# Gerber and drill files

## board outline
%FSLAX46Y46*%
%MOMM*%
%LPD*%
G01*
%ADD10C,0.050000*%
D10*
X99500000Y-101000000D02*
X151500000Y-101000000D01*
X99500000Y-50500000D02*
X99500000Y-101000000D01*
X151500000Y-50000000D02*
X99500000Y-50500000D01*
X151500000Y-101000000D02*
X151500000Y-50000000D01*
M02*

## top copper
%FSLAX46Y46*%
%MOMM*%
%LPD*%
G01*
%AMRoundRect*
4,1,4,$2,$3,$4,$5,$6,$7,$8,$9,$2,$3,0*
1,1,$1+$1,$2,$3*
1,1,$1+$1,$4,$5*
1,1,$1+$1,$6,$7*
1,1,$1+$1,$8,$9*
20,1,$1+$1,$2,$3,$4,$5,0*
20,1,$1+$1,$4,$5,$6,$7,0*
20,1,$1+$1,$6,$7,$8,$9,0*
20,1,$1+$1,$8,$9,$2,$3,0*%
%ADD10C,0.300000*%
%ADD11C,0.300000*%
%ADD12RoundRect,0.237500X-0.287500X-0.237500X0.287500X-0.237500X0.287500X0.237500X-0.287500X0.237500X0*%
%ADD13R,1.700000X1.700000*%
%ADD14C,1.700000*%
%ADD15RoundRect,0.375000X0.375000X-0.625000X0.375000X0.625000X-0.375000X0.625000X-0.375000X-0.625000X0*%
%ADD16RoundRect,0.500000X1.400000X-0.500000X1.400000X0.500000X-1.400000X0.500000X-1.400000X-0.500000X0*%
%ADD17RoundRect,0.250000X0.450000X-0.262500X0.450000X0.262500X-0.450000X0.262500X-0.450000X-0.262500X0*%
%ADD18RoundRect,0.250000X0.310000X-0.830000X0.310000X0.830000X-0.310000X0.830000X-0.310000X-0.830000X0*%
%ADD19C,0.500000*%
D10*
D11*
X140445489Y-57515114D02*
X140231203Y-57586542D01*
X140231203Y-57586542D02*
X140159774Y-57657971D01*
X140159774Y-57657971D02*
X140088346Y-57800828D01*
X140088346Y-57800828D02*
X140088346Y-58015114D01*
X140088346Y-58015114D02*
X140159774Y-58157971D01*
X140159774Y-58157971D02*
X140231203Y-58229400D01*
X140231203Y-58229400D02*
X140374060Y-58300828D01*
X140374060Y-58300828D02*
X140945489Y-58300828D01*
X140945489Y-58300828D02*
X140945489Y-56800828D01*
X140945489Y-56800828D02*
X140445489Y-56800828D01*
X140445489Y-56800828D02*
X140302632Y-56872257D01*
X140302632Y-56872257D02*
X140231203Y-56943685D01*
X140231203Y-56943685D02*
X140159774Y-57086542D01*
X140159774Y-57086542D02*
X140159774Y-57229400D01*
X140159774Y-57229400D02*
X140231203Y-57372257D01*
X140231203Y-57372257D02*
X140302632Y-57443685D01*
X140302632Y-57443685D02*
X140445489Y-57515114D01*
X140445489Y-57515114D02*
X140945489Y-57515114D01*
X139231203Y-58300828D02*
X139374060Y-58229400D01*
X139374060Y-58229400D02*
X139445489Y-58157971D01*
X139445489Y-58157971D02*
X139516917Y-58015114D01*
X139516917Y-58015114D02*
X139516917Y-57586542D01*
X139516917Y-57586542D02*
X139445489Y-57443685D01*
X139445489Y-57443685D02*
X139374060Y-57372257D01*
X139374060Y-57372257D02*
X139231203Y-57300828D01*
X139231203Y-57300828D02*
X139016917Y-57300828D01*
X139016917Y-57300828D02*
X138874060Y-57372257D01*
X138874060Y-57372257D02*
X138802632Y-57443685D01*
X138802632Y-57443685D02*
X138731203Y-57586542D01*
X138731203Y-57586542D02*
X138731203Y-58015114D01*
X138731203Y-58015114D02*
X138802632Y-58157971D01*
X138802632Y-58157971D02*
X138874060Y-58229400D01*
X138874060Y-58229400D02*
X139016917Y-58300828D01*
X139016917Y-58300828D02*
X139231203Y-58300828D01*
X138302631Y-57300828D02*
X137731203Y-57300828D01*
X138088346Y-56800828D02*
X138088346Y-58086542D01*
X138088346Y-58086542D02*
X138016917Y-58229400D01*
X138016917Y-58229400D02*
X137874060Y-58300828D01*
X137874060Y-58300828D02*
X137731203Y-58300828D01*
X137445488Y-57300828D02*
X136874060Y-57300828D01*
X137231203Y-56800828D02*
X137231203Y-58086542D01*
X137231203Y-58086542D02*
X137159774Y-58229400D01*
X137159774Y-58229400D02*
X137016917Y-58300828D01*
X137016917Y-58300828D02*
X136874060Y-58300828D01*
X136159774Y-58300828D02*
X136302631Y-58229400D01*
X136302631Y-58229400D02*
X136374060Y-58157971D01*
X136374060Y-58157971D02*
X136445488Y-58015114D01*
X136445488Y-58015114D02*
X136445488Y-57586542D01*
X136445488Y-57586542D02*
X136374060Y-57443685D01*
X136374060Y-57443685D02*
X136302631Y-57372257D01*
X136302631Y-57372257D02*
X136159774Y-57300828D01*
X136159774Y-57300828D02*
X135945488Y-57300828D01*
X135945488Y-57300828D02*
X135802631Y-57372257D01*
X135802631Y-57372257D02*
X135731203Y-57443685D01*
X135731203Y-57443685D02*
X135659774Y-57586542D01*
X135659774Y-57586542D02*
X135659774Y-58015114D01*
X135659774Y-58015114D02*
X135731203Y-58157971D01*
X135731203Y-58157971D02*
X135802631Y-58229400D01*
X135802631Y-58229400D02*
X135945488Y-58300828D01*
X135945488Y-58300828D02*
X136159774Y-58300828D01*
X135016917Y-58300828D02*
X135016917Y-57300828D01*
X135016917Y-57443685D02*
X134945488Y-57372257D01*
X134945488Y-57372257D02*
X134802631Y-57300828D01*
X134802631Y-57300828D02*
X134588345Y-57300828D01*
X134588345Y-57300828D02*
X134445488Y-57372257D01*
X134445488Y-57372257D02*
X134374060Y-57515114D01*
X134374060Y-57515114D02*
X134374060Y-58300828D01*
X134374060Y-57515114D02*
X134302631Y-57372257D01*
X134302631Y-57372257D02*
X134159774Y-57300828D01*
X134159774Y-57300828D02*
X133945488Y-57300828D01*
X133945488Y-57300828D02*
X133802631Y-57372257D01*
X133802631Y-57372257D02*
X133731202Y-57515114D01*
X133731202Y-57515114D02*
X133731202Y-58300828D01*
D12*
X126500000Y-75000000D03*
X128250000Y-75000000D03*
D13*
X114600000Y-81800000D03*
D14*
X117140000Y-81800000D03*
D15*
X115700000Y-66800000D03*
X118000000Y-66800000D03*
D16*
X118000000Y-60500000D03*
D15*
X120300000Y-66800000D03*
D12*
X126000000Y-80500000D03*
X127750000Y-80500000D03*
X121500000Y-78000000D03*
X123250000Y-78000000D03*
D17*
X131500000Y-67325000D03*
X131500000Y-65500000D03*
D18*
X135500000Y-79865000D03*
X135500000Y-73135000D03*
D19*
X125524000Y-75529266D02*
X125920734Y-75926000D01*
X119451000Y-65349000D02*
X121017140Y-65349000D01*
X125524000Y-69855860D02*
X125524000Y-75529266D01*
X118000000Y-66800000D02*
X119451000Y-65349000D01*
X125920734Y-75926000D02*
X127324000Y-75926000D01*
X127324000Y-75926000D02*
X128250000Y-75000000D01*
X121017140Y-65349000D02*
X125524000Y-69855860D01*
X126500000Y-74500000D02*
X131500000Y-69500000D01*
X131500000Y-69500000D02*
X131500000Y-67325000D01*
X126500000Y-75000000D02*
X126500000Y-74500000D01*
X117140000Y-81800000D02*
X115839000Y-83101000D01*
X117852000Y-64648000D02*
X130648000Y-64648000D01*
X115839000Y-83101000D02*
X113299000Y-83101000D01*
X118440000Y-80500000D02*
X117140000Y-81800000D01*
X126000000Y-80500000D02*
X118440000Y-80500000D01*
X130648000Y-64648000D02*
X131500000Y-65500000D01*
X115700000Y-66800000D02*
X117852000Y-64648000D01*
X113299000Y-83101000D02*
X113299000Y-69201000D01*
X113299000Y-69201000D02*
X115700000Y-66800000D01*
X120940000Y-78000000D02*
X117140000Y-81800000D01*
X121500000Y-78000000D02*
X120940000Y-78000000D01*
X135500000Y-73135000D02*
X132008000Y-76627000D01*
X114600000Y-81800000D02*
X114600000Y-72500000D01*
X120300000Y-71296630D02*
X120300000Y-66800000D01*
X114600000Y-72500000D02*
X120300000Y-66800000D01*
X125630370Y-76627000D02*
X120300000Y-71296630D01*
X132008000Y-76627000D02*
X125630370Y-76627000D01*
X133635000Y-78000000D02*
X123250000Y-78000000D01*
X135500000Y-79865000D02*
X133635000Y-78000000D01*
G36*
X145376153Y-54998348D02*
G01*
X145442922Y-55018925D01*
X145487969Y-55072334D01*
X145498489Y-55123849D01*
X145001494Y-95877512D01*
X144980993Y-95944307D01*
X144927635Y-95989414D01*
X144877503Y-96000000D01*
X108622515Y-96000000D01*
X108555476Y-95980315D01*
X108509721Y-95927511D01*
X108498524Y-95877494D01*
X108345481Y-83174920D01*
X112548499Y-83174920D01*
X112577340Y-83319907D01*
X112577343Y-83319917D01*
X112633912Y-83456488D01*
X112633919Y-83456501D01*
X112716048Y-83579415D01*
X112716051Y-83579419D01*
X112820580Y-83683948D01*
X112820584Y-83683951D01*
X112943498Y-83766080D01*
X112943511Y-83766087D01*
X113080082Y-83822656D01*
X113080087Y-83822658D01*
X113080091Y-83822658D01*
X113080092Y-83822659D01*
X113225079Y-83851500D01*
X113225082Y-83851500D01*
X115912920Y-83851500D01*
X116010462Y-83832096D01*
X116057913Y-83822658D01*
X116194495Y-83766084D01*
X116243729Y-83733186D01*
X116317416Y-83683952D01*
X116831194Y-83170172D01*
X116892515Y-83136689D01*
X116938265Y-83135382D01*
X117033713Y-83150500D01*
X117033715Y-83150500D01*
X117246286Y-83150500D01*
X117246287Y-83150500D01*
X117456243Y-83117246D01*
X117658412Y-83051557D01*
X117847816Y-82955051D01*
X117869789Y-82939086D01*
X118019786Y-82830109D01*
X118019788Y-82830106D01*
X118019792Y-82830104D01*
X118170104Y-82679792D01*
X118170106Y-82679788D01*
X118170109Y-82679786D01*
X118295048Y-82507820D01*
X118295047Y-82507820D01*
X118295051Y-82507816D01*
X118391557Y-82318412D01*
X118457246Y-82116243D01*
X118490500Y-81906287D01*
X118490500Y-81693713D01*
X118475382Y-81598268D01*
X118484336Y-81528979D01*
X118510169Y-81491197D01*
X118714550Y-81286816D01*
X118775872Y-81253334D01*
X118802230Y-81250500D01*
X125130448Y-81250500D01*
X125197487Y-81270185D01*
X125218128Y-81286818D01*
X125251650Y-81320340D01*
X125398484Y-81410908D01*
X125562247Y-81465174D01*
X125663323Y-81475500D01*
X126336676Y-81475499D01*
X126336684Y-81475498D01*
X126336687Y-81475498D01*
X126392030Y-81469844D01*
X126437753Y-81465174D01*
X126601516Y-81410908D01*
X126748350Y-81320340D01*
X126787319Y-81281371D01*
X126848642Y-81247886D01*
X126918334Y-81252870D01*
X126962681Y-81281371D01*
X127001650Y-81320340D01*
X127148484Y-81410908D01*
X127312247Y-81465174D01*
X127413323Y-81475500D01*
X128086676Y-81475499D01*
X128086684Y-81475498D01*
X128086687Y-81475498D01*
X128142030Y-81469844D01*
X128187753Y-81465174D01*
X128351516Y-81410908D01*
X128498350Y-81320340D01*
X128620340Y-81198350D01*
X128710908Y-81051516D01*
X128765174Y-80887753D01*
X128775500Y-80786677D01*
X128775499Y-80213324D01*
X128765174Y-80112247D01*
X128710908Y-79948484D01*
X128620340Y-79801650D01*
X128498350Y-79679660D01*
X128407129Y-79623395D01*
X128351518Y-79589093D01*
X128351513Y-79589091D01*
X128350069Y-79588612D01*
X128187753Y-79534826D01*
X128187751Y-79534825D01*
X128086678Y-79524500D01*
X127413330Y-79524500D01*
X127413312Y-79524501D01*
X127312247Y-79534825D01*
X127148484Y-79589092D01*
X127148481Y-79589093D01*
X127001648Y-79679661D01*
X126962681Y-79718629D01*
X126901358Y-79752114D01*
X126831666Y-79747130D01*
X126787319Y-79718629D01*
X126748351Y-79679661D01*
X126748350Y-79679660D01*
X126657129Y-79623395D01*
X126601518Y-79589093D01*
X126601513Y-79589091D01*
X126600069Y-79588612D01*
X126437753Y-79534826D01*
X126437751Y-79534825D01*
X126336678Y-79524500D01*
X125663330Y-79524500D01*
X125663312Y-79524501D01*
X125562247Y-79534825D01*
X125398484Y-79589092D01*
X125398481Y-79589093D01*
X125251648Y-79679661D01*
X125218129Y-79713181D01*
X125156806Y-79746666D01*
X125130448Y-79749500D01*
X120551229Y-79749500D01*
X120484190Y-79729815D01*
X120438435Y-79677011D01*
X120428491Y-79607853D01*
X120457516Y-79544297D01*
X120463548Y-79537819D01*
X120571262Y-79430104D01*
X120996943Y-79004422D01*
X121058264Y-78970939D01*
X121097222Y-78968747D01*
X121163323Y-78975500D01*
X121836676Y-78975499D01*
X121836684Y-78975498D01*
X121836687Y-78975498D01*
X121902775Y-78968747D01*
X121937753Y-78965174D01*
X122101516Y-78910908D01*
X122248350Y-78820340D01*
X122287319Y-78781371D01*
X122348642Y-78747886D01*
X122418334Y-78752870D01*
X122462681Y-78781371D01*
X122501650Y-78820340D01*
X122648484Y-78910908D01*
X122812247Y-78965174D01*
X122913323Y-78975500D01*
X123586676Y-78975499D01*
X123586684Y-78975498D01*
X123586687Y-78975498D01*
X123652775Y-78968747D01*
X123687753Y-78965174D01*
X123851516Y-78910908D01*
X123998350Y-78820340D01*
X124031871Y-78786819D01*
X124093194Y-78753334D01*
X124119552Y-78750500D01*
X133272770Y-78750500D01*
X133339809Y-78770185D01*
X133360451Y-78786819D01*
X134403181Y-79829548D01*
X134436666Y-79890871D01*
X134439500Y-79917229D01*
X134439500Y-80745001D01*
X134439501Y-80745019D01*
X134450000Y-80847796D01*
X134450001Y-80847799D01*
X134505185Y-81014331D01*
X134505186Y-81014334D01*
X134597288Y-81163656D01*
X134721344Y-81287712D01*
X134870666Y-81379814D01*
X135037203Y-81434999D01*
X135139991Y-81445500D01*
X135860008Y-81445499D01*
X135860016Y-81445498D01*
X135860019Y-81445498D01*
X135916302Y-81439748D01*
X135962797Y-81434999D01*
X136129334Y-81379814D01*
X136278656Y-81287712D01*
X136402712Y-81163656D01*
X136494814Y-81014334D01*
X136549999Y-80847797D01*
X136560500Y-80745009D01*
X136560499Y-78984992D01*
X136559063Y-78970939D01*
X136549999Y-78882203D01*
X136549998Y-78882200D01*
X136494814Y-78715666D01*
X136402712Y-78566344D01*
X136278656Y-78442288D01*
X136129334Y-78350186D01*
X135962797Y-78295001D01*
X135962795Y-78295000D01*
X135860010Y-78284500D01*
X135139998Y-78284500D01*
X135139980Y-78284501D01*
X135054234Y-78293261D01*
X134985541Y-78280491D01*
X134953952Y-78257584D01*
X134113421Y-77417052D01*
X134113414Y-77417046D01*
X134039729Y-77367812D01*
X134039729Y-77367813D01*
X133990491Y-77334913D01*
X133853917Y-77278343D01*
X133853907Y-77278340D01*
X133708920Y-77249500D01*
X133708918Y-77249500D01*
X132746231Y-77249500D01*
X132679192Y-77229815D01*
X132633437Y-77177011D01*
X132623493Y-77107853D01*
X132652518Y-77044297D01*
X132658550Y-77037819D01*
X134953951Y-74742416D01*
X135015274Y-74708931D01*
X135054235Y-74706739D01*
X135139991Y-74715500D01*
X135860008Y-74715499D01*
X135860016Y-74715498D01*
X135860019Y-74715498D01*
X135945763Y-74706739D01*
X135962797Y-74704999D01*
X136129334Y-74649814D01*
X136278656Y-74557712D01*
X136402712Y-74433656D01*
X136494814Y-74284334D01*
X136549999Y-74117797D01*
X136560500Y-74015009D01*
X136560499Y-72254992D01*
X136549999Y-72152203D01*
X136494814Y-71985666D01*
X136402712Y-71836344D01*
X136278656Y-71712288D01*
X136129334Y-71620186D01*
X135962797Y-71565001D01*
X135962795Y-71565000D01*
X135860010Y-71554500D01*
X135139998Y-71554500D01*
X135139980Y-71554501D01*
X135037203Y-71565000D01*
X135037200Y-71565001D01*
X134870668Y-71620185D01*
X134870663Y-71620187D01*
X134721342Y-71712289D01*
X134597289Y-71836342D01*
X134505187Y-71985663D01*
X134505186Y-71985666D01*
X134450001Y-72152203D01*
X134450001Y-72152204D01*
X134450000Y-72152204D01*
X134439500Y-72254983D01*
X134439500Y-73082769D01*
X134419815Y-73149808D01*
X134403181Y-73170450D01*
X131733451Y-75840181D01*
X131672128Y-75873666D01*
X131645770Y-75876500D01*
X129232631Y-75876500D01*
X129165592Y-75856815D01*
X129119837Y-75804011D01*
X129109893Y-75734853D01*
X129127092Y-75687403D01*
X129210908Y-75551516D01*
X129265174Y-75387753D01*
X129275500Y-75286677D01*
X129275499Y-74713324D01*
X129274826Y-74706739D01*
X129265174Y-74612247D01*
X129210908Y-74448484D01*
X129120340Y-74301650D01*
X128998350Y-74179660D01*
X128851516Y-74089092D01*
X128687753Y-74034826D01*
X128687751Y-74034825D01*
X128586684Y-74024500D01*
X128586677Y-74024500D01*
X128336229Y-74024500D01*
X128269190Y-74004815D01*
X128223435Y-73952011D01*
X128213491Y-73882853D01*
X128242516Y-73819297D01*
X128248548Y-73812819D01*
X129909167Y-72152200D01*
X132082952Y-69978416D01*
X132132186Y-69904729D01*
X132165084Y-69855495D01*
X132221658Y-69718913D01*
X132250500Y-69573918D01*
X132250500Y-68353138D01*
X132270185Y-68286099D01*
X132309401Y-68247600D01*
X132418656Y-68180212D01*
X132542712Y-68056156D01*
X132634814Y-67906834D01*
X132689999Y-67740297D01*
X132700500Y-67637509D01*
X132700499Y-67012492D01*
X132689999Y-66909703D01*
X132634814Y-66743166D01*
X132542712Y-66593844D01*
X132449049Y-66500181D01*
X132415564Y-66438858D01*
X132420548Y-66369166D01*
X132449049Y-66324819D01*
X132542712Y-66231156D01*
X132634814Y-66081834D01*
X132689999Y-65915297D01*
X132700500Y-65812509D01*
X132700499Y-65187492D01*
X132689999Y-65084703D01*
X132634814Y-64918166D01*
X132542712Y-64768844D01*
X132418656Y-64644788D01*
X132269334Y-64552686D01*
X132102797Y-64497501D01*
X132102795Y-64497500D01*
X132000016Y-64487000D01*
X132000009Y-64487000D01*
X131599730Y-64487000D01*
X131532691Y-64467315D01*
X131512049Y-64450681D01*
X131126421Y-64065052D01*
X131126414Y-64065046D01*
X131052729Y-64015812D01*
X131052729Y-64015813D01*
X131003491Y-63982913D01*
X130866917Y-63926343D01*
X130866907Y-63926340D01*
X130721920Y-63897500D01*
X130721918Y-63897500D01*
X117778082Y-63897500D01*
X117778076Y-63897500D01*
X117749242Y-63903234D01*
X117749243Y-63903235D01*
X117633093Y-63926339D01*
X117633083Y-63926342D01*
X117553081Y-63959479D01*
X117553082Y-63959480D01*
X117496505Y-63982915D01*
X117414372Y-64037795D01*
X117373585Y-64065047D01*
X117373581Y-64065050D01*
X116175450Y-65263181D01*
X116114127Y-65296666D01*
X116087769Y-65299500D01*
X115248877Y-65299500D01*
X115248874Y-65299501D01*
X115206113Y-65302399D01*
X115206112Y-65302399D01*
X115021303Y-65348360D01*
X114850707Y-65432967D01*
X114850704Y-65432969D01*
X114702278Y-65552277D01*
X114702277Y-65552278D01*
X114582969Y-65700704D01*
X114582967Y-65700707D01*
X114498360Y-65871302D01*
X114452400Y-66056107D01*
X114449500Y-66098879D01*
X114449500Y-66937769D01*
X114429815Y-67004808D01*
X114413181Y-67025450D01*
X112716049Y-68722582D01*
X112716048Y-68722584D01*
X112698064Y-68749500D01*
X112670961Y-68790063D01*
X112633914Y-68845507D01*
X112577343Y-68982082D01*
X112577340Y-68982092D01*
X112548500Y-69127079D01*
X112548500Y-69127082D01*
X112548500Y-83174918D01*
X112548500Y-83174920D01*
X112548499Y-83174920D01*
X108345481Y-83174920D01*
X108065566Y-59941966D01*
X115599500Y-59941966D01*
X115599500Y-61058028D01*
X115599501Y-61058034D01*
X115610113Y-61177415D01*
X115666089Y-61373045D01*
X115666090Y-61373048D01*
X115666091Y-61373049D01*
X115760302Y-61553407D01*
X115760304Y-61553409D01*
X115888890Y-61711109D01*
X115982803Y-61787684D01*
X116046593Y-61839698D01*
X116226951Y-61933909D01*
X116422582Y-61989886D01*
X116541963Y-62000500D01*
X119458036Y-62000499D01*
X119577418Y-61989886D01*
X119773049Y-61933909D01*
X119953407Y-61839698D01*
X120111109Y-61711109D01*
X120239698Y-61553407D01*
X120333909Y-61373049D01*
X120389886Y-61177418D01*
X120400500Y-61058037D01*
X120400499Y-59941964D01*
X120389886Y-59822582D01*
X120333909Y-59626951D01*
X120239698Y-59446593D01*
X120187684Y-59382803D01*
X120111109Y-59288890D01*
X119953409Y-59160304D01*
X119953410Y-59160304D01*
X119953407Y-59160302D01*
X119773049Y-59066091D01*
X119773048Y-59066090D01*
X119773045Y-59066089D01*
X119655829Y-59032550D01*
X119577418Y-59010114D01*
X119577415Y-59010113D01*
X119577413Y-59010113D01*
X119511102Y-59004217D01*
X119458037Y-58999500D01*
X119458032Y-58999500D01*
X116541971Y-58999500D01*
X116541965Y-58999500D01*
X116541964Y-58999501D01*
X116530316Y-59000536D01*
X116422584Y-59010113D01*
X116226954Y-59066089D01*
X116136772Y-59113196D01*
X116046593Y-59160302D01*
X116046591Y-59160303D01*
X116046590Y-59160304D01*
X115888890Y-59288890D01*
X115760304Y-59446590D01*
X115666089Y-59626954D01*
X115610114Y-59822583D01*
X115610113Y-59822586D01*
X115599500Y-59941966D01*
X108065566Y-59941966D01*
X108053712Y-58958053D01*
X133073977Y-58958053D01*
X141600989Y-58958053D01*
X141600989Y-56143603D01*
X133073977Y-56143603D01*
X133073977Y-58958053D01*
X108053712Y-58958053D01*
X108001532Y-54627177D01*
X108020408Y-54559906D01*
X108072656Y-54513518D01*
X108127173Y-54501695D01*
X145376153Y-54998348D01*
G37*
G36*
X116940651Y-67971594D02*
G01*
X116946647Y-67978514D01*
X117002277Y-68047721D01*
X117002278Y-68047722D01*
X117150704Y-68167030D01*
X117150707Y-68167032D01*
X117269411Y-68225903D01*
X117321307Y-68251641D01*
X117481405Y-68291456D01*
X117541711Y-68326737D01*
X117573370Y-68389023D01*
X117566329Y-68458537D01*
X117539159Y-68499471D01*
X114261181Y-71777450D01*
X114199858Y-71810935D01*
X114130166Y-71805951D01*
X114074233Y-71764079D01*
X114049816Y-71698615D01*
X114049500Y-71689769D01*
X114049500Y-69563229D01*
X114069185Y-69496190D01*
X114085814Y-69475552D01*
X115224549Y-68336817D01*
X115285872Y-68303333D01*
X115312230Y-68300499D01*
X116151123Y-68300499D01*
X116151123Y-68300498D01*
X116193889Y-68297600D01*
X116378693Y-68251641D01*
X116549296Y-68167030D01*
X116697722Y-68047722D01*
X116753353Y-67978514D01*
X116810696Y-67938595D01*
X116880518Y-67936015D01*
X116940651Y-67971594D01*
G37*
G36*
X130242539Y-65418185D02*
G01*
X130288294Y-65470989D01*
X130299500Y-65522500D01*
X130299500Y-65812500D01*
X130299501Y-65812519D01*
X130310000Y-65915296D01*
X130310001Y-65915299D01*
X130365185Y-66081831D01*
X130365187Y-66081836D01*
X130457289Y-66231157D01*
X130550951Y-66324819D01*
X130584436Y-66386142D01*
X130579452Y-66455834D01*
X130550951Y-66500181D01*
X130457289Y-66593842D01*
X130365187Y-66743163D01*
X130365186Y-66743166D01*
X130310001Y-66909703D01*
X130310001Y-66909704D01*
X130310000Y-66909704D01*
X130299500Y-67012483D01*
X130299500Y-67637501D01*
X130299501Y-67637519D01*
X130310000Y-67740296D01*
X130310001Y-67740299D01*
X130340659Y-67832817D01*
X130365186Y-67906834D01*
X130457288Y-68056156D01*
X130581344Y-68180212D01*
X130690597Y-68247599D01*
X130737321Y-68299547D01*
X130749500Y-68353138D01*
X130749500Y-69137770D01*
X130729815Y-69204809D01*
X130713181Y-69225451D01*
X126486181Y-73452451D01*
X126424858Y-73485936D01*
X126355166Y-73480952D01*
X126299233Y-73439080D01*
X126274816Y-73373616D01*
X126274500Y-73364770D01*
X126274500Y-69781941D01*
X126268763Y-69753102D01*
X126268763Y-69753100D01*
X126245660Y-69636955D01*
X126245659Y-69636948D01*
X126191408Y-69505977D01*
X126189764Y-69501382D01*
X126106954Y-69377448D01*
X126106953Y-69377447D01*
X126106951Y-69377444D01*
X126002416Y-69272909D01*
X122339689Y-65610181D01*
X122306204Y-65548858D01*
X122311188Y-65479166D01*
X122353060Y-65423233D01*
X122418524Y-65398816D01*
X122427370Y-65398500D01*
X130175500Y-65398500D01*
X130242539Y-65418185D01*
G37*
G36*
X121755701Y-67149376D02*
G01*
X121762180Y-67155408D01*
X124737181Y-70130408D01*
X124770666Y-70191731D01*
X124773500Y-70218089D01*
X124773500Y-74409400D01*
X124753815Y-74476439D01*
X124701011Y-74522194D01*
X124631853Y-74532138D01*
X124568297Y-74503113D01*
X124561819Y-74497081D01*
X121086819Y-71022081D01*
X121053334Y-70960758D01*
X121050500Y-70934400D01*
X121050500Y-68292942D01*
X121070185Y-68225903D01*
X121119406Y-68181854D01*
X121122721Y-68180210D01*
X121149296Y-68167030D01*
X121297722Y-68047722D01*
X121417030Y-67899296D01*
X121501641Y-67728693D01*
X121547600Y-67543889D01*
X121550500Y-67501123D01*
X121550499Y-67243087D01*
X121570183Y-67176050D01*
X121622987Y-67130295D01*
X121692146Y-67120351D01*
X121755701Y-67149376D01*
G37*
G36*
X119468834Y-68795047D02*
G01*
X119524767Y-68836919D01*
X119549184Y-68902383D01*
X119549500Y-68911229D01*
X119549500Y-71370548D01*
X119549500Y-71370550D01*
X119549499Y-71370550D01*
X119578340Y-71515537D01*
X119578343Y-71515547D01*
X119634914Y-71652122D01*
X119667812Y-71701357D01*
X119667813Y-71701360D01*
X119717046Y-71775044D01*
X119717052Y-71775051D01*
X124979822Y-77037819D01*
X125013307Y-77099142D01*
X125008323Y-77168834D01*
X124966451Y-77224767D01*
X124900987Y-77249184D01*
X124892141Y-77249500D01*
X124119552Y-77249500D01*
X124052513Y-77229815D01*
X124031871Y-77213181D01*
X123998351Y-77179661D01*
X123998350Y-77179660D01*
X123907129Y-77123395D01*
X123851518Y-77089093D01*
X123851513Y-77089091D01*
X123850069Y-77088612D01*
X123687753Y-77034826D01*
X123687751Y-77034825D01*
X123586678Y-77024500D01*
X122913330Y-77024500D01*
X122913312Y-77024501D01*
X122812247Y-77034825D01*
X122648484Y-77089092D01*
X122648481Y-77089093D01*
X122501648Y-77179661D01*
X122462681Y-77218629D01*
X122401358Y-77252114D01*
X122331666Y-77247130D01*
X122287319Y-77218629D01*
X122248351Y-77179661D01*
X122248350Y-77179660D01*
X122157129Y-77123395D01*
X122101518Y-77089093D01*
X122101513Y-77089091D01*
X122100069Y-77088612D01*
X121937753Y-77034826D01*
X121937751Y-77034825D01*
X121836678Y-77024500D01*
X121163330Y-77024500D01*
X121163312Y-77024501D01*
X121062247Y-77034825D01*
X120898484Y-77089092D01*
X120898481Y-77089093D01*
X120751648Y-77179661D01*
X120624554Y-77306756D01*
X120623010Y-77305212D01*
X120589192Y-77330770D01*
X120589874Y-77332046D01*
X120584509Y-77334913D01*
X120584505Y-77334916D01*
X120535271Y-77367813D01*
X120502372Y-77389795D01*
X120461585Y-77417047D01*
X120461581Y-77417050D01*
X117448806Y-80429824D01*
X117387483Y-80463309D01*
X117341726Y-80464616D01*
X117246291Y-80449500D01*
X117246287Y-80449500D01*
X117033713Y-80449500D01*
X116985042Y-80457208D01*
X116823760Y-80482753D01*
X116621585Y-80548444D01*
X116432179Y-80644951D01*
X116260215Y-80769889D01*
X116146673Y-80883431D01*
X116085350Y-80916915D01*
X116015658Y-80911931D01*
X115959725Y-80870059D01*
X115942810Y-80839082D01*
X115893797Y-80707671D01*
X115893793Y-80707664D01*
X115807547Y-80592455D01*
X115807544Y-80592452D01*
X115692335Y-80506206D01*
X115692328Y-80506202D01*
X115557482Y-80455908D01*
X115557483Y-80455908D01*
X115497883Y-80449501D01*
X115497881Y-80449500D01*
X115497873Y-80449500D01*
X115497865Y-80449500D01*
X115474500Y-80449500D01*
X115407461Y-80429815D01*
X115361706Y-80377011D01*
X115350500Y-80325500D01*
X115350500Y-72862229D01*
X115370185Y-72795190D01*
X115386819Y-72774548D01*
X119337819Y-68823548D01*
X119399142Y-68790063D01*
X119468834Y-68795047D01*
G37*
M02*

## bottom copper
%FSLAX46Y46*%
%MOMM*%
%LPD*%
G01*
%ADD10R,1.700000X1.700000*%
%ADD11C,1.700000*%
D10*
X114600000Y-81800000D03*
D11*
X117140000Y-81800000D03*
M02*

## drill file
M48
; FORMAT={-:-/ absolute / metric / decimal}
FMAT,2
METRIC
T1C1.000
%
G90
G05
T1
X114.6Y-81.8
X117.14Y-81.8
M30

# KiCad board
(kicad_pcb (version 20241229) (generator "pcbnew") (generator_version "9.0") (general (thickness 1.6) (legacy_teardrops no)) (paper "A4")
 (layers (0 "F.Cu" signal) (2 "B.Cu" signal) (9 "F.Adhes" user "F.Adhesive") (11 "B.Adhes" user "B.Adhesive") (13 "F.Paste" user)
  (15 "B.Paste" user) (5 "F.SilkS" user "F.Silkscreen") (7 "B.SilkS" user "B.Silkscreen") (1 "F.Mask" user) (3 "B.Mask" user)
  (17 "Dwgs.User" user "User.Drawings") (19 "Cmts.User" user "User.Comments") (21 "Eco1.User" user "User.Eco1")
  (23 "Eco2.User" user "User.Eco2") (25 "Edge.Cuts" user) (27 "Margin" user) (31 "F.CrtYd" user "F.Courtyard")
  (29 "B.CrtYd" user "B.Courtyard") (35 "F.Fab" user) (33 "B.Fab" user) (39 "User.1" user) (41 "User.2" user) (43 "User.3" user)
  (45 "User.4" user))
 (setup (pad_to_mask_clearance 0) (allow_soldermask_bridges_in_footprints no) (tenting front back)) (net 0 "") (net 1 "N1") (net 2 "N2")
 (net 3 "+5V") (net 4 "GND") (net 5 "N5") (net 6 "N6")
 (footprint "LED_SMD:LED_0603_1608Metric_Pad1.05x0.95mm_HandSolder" (layer "F.Cu") (at 127.375 75)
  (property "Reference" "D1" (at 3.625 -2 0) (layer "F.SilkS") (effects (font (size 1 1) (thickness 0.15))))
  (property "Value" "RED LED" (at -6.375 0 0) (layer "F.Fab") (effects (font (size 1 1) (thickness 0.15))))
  (pad "1" smd roundrect (at -0.875 0) (size 1.05 0.95) (layers "F.Cu" "F.Mask" "F.Paste") (roundrect_rratio 0.25) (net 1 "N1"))
  (pad "2" smd roundrect (at 0.875 0) (size 1.05 0.95) (layers "F.Cu" "F.Mask" "F.Paste") (roundrect_rratio 0.25) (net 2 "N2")))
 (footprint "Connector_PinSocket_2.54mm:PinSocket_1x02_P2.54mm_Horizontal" (layer "F.Cu") (at 114.6 81.8 90)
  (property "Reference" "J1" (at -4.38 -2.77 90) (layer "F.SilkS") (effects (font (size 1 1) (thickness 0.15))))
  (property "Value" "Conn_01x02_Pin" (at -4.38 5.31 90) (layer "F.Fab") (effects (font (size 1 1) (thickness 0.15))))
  (pad "1" thru_hole rect (at 0 0 90) (size 1.7 1.7) (drill 1) (layers "*.Cu" "*.Mask") (remove_unused_layers no) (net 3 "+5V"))
  (pad "2" thru_hole circle (at 0 2.54 90) (size 1.7 1.7) (drill 1) (layers "*.Cu" "*.Mask") (remove_unused_layers no) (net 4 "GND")))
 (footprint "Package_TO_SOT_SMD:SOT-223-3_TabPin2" (layer "F.Cu") (at 118 63.65 90)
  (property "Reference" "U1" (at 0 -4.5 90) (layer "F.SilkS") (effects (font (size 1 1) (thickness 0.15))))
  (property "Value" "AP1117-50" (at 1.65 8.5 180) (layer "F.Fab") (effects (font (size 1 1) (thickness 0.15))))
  (pad "1" smd roundrect (at -3.15 -2.3 90) (size 2 1.5) (layers "F.Cu" "F.Mask" "F.Paste") (roundrect_rratio 0.25) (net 4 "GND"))
  (pad "2" smd roundrect (at -3.15 0 90) (size 2 1.5) (layers "F.Cu" "F.Mask" "F.Paste") (roundrect_rratio 0.25) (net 2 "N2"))
  (pad "2" smd roundrect (at 3.15 0 90) (size 2 3.8) (layers "F.Cu" "F.Mask" "F.Paste") (roundrect_rratio 0.25) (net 2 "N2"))
  (pad "3" smd roundrect (at -3.15 2.3 90) (size 2 1.5) (layers "F.Cu" "F.Mask" "F.Paste") (roundrect_rratio 0.25) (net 3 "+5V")))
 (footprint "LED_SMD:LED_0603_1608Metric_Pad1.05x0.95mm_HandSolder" (layer "F.Cu") (at 126.875 80.5)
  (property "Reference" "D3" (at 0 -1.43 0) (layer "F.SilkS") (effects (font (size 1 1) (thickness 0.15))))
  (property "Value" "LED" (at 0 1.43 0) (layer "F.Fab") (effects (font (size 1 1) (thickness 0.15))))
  (pad "1" smd roundrect (at -0.875 0) (size 1.05 0.95) (layers "F.Cu" "F.Mask" "F.Paste") (roundrect_rratio 0.25) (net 4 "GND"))
  (pad "2" smd roundrect (at 0.875 0) (size 1.05 0.95) (layers "F.Cu" "F.Mask" "F.Paste") (roundrect_rratio 0.25) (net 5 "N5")))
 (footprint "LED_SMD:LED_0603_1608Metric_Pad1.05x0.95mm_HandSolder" (layer "F.Cu") (at 122.375 78)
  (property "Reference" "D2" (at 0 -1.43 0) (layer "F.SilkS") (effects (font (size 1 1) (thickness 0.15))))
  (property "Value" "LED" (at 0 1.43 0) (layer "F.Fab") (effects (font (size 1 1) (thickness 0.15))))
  (pad "1" smd roundrect (at -0.875 0) (size 1.05 0.95) (layers "F.Cu" "F.Mask" "F.Paste") (roundrect_rratio 0.25) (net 4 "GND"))
  (pad "2" smd roundrect (at 0.875 0) (size 1.05 0.95) (layers "F.Cu" "F.Mask" "F.Paste") (roundrect_rratio 0.25) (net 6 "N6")))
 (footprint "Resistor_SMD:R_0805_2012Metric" (layer "F.Cu") (at 131.5 66.4125 90)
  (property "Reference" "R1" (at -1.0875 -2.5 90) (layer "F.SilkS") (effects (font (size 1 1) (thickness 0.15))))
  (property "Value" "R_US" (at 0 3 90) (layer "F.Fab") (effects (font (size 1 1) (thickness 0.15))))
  (pad "1" smd roundrect (at -0.9125 0 90) (size 1.025 1.4) (layers "F.Cu" "F.Mask" "F.Paste") (roundrect_rratio 0.243902) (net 1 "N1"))
  (pad "2" smd roundrect (at 0.9125 0 90) (size 1.025 1.4) (layers "F.Cu" "F.Mask" "F.Paste") (roundrect_rratio 0.243902) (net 4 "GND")))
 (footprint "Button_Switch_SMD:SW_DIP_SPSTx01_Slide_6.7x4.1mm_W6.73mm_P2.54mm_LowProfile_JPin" (layer "F.Cu") (at 135.5 76.5 90)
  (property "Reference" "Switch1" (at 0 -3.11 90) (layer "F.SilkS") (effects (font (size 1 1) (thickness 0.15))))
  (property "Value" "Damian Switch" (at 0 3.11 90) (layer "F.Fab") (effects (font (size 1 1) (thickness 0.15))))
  (pad "1" smd roundrect (at -3.365 0 90) (size 2.16 1.12) (layers "F.Cu" "F.Mask" "F.Paste") (roundrect_rratio 0.223214) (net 6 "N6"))
  (pad "2" smd roundrect (at 3.365 0 90) (size 2.16 1.12) (layers "F.Cu" "F.Mask" "F.Paste") (roundrect_rratio 0.223214) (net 3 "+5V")))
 (gr_line (start 99.5 101) (end 151.5 101) (stroke (width 0.05) (type default)) (layer "Edge.Cuts"))
 (gr_line (start 99.5 50.5) (end 99.5 101) (stroke (width 0.05) (type default)) (layer "Edge.Cuts"))
 (gr_line (start 151.5 50) (end 99.5 50.5) (stroke (width 0.05) (type default)) (layer "Edge.Cuts"))
 (gr_line (start 151.5 101) (end 151.5 50) (stroke (width 0.05) (type default)) (layer "Edge.Cuts"))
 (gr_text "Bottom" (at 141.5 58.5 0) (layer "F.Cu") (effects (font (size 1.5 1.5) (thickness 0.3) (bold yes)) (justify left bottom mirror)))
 (segment (start 125.524 75.529266) (end 125.920734 75.926) (width 0.5) (layer "F.Cu") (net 2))
 (segment (start 119.451 65.349) (end 121.01714 65.349) (width 0.5) (layer "F.Cu") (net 2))
 (segment (start 125.524 69.85586) (end 125.524 75.529266) (width 0.5) (layer "F.Cu") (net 2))
 (segment (start 118 66.8) (end 119.451 65.349) (width 0.5) (layer "F.Cu") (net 2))
 (segment (start 125.920734 75.926) (end 127.324 75.926) (width 0.5) (layer "F.Cu") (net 2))
 (segment (start 127.324 75.926) (end 128.25 75) (width 0.5) (layer "F.Cu") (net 2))
 (segment (start 121.01714 65.349) (end 125.524 69.85586) (width 0.5) (layer "F.Cu") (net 2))
 (segment (start 126.5 74.5) (end 131.5 69.5) (width 0.5) (layer "F.Cu") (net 1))
 (segment (start 131.5 69.5) (end 131.5 67.325) (width 0.5) (layer "F.Cu") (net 1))
 (segment (start 126.5 75) (end 126.5 74.5) (width 0.5) (layer "F.Cu") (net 1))
 (segment (start 117.14 81.8) (end 115.839 83.101) (width 0.5) (layer "F.Cu") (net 4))
 (segment (start 117.852 64.648) (end 130.648 64.648) (width 0.5) (layer "F.Cu") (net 4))
 (segment (start 115.839 83.101) (end 113.299 83.101) (width 0.5) (layer "F.Cu") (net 4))
 (segment (start 118.44 80.5) (end 117.14 81.8) (width 0.5) (layer "F.Cu") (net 4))
 (segment (start 126 80.5) (end 118.44 80.5) (width 0.5) (layer "F.Cu") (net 4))
 (segment (start 130.648 64.648) (end 131.5 65.5) (width 0.5) (layer "F.Cu") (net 4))
 (segment (start 115.7 66.8) (end 117.852 64.648) (width 0.5) (layer "F.Cu") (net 4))
 (segment (start 113.299 83.101) (end 113.299 69.201) (width 0.5) (layer "F.Cu") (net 4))
 (segment (start 113.299 69.201) (end 115.7 66.8) (width 0.5) (layer "F.Cu") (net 4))
 (segment (start 120.94 78) (end 117.14 81.8) (width 0.5) (layer "F.Cu") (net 4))
 (segment (start 121.5 78) (end 120.94 78) (width 0.5) (layer "F.Cu") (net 4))
 (segment (start 135.5 73.135) (end 132.008 76.627) (width 0.5) (layer "F.Cu") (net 3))
 (segment (start 114.6 81.8) (end 114.6 72.5) (width 0.5) (layer "F.Cu") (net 3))
 (segment (start 120.3 71.29663) (end 120.3 66.8) (width 0.5) (layer "F.Cu") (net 3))
 (segment (start 114.6 72.5) (end 120.3 66.8) (width 0.5) (layer "F.Cu") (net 3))
 (segment (start 125.63037 76.627) (end 120.3 71.29663) (width 0.5) (layer "F.Cu") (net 3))
 (segment (start 132.008 76.627) (end 125.63037 76.627) (width 0.5) (layer "F.Cu") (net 3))
 (segment (start 133.635 78) (end 123.25 78) (width 0.5) (layer "F.Cu") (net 6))
 (segment (start 135.5 79.865) (end 133.635 78) (width 0.5) (layer "F.Cu") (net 6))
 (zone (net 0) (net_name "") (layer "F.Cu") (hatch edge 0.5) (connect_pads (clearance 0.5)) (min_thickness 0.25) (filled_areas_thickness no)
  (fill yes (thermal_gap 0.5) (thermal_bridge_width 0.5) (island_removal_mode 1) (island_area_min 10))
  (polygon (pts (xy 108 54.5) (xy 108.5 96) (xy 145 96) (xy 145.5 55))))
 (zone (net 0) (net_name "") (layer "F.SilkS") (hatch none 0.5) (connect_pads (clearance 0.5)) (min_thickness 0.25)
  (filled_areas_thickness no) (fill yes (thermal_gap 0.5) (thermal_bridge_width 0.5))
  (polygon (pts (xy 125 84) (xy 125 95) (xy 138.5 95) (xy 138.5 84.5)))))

